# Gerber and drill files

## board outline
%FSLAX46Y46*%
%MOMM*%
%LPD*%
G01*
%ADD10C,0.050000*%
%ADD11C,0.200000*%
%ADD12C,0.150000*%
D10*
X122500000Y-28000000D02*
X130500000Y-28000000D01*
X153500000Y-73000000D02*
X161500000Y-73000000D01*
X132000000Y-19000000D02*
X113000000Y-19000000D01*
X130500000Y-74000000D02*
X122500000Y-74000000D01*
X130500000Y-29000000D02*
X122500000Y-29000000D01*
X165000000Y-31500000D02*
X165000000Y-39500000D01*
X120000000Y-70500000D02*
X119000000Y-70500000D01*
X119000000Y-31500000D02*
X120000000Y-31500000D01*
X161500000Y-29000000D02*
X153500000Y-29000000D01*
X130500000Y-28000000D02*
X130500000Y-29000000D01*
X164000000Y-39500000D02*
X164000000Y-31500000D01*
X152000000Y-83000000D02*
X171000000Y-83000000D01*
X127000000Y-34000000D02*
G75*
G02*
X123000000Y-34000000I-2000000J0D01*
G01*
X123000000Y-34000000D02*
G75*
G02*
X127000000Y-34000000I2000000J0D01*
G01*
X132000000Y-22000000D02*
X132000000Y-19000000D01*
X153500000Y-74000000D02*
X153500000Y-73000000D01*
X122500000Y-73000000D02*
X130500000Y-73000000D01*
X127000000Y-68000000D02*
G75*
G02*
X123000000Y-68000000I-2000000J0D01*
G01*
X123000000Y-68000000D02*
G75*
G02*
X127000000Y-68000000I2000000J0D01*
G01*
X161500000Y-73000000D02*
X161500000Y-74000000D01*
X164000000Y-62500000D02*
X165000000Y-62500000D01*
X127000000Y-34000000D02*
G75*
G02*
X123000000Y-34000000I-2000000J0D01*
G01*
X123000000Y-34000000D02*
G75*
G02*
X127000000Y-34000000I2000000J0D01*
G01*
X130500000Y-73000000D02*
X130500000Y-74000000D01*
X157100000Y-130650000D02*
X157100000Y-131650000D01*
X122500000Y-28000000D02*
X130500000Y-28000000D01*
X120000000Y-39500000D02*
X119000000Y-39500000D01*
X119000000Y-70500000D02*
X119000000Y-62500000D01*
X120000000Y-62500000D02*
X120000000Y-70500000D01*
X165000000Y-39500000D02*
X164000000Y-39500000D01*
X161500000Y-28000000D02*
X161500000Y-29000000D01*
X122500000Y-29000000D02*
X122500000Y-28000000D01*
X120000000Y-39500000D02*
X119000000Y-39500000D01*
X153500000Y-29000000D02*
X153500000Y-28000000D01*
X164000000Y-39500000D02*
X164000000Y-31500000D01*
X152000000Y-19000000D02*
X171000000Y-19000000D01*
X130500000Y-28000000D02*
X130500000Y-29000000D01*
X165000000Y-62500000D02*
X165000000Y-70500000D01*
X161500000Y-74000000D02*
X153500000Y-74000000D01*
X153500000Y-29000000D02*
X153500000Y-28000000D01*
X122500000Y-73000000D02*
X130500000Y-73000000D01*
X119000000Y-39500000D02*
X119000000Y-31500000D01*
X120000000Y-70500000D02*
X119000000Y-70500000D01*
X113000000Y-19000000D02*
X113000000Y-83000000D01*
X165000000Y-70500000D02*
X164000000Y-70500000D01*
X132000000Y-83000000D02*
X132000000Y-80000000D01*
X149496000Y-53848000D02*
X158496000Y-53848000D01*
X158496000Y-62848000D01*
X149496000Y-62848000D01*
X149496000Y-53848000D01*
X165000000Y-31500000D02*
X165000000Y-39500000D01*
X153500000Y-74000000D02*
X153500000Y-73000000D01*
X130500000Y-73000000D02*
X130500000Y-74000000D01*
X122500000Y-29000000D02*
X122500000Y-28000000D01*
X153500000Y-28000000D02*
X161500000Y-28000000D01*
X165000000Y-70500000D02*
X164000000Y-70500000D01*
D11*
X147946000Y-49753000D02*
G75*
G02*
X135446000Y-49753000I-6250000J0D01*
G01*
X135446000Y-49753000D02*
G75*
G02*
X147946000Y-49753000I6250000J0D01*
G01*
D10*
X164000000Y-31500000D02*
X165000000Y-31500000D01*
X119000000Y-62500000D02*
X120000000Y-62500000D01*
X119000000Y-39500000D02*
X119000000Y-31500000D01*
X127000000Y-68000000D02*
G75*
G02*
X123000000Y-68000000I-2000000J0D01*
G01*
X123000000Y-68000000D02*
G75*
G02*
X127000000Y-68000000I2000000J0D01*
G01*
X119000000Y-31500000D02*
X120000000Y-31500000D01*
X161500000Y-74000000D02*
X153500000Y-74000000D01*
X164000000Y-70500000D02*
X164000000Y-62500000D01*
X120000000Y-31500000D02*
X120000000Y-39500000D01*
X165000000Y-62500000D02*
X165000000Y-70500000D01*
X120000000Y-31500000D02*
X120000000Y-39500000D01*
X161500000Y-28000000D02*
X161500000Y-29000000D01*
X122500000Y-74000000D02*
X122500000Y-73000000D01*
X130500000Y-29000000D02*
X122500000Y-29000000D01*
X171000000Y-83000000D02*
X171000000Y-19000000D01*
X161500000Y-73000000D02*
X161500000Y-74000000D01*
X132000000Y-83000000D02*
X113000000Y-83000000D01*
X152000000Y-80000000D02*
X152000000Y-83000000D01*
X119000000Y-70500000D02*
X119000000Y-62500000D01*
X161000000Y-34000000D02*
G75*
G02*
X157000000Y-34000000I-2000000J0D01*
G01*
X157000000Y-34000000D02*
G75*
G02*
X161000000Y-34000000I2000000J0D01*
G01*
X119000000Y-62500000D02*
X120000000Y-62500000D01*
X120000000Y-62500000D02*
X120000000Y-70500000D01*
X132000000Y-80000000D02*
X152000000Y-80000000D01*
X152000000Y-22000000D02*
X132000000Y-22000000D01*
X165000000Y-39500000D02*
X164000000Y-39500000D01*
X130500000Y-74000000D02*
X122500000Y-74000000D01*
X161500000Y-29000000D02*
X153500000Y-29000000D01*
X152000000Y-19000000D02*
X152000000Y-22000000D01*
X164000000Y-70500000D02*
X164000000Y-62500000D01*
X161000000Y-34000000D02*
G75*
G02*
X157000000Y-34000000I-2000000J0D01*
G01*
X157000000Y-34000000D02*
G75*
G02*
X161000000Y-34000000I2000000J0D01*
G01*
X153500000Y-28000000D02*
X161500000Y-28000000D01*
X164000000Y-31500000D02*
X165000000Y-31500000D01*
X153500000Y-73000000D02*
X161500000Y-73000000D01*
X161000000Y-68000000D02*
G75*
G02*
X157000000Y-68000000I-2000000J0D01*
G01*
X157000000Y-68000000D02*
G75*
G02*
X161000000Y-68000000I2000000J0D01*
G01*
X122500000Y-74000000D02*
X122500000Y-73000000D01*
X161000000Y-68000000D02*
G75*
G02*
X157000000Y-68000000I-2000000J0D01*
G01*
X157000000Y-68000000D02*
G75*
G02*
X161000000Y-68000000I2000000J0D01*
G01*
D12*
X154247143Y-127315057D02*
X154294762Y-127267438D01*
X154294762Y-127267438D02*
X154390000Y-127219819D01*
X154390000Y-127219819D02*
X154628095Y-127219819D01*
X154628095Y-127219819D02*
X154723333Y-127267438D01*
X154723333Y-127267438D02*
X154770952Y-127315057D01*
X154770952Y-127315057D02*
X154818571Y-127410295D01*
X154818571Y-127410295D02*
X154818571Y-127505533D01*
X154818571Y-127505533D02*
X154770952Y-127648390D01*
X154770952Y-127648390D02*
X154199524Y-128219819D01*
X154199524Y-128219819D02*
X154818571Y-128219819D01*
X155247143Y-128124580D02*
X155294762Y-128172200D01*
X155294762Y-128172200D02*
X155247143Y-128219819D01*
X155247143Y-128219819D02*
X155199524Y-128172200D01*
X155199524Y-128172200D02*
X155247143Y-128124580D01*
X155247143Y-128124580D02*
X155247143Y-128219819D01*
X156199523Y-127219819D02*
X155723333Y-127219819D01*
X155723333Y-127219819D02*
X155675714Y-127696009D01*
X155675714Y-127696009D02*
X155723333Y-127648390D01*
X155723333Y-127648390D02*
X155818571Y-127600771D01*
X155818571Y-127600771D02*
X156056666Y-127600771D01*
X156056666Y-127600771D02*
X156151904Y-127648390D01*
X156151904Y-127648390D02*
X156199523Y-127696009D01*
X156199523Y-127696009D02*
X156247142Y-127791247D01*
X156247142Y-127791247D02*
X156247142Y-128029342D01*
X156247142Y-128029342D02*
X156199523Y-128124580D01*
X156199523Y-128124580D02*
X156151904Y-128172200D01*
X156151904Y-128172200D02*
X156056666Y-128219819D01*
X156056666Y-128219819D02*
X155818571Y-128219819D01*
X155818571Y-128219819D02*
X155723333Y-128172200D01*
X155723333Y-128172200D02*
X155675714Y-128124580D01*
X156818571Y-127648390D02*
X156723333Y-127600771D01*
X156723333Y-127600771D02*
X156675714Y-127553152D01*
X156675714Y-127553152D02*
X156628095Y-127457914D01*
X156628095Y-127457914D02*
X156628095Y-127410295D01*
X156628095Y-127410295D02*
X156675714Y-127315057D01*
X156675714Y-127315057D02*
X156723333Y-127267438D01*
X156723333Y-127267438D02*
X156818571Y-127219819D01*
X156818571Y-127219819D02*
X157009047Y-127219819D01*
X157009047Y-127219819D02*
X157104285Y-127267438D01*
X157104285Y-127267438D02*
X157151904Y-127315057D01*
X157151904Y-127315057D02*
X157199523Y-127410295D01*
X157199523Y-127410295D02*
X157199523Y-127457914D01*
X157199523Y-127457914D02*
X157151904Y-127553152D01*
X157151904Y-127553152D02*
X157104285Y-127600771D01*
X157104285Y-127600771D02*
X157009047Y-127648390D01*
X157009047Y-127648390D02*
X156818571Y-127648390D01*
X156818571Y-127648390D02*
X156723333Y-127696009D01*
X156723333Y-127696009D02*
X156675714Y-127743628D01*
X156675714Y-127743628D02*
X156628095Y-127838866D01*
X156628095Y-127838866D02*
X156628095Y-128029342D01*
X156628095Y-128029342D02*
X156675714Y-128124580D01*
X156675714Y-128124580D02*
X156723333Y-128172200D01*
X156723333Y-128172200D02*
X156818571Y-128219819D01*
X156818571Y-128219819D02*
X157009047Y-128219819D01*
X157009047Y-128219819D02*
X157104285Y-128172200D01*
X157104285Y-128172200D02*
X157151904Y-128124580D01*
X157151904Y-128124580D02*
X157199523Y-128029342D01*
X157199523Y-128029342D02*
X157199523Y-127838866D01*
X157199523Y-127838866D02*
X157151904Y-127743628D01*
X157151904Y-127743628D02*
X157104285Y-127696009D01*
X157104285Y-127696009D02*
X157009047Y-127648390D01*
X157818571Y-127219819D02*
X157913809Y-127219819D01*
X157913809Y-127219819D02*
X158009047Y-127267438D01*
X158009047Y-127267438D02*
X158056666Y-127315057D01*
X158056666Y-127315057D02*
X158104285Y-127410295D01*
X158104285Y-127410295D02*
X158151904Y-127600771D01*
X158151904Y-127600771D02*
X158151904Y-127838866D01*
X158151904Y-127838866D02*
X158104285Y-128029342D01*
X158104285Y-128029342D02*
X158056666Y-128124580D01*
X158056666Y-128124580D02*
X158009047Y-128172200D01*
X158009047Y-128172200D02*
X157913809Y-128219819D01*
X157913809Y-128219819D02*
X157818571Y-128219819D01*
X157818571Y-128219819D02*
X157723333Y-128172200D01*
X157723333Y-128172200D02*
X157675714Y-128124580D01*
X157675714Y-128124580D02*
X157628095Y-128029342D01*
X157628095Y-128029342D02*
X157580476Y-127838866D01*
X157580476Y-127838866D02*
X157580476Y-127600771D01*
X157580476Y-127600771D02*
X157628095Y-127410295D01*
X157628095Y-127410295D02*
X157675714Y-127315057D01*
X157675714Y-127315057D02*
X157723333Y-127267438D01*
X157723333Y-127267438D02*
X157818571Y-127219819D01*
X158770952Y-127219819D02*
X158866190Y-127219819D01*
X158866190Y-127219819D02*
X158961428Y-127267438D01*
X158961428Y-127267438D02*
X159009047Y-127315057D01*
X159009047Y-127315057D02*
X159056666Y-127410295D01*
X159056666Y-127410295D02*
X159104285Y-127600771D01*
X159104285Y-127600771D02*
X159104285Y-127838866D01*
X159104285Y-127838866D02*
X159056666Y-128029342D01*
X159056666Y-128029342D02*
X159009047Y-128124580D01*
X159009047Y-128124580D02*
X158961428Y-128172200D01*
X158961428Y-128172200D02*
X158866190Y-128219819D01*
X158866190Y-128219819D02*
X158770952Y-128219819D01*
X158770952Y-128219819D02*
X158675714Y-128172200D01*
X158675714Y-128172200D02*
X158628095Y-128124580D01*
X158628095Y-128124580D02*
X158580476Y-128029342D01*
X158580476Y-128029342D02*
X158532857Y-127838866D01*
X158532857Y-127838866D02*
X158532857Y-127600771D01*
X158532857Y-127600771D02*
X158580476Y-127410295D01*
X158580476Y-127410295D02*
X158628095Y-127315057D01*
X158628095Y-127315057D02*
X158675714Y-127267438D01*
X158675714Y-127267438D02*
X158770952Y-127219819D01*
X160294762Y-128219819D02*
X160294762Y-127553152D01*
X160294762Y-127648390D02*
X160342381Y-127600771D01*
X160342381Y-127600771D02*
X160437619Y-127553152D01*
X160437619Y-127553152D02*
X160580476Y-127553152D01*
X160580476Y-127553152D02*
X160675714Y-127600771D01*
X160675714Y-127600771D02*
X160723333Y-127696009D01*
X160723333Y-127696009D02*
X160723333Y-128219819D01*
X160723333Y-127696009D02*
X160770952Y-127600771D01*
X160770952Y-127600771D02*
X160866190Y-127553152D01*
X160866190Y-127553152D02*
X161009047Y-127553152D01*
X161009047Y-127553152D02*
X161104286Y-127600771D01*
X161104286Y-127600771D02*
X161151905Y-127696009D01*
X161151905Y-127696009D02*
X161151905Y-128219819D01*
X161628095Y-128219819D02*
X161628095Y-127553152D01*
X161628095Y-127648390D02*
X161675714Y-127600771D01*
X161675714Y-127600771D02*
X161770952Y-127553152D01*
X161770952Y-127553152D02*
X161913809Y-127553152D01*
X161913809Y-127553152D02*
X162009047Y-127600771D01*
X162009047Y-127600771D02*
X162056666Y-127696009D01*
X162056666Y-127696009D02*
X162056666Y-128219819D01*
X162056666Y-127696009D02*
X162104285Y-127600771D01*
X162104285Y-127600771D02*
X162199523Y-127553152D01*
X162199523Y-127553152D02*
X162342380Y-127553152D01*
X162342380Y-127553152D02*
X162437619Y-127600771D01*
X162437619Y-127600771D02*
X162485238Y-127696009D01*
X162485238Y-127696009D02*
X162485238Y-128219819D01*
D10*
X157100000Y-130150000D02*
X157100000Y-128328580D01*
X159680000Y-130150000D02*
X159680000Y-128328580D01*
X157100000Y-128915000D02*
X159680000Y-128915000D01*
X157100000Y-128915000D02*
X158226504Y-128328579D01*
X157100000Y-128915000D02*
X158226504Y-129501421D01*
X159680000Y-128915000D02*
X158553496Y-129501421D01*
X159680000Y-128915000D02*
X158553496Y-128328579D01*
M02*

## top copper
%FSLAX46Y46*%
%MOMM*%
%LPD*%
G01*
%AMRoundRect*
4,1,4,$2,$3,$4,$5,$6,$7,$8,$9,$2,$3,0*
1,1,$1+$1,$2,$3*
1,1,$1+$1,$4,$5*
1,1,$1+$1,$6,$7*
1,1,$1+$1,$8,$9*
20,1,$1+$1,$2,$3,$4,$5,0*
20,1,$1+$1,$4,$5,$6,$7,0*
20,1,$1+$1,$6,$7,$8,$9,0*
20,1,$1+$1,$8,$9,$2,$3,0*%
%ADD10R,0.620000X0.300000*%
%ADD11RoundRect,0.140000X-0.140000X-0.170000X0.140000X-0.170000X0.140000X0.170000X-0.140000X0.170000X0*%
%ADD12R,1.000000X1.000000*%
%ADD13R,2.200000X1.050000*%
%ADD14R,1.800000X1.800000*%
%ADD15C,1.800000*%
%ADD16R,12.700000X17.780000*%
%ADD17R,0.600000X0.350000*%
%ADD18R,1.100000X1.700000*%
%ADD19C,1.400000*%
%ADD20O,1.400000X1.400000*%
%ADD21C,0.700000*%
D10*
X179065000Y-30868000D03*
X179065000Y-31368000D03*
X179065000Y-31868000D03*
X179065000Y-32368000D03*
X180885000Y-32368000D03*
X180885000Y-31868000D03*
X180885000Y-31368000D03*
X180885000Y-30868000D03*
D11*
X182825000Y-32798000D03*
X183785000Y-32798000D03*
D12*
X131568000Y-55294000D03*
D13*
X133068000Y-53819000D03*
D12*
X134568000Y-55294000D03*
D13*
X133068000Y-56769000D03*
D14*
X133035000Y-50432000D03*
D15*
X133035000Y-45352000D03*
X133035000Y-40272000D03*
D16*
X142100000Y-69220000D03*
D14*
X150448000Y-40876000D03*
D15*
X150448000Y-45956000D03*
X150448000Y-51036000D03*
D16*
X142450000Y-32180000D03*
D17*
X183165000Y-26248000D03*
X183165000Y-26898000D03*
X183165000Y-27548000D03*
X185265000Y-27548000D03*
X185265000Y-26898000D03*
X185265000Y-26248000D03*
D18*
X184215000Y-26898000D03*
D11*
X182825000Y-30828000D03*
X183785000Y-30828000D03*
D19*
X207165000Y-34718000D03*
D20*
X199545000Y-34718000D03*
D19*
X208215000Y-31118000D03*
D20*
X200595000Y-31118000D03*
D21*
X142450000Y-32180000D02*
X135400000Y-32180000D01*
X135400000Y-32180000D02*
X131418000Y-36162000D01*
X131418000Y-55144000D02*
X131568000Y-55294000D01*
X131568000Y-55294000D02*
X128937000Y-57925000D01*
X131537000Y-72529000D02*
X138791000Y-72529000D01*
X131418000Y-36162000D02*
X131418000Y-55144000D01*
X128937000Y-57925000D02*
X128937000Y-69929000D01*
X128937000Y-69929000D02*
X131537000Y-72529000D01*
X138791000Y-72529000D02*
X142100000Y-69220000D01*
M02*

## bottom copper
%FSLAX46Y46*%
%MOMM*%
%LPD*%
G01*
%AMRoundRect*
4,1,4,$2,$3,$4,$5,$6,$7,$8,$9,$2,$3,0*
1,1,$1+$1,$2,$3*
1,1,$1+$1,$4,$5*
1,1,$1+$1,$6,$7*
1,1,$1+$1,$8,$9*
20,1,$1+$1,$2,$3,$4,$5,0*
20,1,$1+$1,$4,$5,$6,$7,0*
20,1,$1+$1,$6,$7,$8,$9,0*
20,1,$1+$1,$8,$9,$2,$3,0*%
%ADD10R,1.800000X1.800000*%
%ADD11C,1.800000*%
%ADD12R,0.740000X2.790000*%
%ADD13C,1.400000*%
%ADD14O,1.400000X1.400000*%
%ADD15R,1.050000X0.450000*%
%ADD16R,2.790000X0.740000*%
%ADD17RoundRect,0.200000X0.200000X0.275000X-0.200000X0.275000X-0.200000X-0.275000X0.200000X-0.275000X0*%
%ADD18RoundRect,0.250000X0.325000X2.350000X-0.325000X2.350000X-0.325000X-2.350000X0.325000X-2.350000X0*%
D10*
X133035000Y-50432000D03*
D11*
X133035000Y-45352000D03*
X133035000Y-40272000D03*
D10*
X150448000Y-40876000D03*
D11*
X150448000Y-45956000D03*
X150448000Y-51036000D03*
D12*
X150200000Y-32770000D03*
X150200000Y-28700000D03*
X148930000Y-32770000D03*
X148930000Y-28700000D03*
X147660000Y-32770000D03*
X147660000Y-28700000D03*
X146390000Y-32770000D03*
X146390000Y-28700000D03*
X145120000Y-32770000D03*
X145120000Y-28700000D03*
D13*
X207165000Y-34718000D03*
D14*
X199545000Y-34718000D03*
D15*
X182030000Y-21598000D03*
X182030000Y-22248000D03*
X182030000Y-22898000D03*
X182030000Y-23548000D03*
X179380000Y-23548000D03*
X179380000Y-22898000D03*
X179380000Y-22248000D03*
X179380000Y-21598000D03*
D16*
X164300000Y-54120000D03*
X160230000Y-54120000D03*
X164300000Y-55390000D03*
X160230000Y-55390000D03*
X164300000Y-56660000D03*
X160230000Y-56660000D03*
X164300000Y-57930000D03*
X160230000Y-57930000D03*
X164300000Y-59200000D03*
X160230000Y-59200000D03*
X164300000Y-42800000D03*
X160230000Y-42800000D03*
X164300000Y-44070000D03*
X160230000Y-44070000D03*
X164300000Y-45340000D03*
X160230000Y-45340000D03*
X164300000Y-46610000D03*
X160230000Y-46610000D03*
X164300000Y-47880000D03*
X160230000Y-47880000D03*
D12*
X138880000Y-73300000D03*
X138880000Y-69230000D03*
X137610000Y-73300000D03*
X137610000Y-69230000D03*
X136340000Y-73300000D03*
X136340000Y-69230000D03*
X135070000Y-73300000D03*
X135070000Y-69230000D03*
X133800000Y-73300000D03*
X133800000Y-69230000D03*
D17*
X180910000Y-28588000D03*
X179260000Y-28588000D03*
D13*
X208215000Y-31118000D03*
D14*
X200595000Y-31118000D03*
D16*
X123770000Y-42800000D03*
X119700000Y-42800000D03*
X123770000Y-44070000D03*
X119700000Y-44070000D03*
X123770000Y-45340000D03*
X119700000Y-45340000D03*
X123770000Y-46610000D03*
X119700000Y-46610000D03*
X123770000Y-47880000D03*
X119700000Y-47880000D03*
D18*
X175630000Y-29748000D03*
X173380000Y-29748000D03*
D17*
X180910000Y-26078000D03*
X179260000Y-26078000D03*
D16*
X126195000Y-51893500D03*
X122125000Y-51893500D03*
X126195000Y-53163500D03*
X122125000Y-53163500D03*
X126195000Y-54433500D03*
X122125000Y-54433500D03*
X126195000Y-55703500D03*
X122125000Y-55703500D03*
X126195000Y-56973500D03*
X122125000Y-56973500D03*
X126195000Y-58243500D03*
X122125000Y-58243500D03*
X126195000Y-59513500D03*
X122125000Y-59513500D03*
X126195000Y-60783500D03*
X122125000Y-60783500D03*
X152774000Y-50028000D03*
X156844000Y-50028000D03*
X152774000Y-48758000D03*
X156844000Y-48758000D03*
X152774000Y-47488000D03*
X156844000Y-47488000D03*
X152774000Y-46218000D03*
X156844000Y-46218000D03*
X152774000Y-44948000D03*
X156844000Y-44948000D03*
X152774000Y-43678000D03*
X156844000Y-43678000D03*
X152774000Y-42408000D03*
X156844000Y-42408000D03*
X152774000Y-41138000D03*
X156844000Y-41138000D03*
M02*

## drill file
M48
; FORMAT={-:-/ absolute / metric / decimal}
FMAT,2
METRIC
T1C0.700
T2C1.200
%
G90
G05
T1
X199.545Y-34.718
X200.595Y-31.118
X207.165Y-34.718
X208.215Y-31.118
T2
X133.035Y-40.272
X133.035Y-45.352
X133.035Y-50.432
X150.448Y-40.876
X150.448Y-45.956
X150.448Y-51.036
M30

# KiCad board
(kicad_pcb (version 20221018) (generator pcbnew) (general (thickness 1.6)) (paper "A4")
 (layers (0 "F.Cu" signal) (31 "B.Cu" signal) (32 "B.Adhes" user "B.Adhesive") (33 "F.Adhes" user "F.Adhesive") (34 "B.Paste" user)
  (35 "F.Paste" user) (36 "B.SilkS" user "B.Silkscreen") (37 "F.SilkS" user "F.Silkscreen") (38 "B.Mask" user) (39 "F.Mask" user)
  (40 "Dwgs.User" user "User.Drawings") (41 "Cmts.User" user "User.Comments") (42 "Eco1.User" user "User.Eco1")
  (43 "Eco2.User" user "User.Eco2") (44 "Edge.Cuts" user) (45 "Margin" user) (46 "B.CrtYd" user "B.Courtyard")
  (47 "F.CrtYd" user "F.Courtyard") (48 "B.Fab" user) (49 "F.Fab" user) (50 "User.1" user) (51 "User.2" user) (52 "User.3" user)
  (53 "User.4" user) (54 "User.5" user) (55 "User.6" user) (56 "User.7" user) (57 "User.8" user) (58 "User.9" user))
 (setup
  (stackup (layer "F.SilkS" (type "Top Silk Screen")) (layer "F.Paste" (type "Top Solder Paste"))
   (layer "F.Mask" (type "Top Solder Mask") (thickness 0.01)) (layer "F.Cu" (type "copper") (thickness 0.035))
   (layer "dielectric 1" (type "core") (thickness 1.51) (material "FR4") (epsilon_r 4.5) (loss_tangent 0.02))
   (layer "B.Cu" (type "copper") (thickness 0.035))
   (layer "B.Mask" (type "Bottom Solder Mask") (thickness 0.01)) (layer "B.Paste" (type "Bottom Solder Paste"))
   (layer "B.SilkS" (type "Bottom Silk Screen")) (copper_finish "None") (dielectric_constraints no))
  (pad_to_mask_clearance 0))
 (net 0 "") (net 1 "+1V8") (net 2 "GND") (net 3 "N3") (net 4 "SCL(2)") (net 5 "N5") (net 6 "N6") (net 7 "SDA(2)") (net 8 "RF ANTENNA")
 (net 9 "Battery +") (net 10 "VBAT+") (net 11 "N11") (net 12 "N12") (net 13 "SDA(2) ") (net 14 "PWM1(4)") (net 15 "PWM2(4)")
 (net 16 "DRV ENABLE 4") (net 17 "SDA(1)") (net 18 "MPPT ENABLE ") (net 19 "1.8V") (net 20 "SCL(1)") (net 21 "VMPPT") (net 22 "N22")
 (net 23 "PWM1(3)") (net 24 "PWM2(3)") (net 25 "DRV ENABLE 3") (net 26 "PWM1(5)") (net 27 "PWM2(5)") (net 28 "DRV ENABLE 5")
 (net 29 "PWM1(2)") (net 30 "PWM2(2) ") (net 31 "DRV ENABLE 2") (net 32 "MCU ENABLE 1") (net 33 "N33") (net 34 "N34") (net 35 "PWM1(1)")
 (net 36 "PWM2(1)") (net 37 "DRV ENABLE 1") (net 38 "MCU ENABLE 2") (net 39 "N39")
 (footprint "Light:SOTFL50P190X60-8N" (layer "F.Cu") (at 179.975 31.618)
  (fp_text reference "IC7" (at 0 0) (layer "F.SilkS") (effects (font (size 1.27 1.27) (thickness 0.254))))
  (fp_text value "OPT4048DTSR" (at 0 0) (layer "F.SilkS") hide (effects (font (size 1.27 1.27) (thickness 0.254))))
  (pad "1" smd rect (at -0.91 -0.75 90) (size 0.3 0.62) (layers "F.Cu" "F.Paste" "F.Mask") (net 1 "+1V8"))
  (pad "2" smd rect (at -0.91 -0.25 90) (size 0.3 0.62) (layers "F.Cu" "F.Paste" "F.Mask") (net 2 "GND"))
  (pad "3" smd rect (at -0.91 0.25 90) (size 0.3 0.62) (layers "F.Cu" "F.Paste" "F.Mask") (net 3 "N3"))
  (pad "4" smd rect (at -0.91 0.75 90) (size 0.3 0.62) (layers "F.Cu" "F.Paste" "F.Mask") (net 2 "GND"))
  (pad "5" smd rect (at 0.91 0.75 90) (size 0.3 0.62) (layers "F.Cu" "F.Paste" "F.Mask") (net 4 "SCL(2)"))
  (pad "6" smd rect (at 0.91 0.25 90) (size 0.3 0.62) (layers "F.Cu" "F.Paste" "F.Mask") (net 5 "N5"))
  (pad "7" smd rect (at 0.91 -0.25 90) (size 0.3 0.62) (layers "F.Cu" "F.Paste" "F.Mask") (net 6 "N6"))
  (pad "8" smd rect (at 0.91 -0.75 90) (size 0.3 0.62) (layers "F.Cu" "F.Paste" "F.Mask") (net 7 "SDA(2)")))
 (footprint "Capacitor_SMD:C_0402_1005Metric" (layer "F.Cu") (at 183.305 32.798)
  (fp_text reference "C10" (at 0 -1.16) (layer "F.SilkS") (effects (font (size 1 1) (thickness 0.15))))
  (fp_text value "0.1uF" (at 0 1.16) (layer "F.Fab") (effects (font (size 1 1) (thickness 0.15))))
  (pad "1" smd roundrect (at -0.48 0) (size 0.56 0.62) (layers "F.Cu" "F.Paste" "F.Mask") (roundrect_rratio 0.25) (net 2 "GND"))
  (pad "2" smd roundrect (at 0.48 0) (size 0.56 0.62) (layers "F.Cu" "F.Paste" "F.Mask") (roundrect_rratio 0.25) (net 1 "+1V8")))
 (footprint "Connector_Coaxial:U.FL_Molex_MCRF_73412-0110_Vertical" (layer "F.Cu") (at 133.068 55.294 -90)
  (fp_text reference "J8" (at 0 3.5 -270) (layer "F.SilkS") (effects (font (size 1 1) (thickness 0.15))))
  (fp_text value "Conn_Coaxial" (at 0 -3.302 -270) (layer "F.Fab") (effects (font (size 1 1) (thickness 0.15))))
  (pad "1" smd rect (at 0 1.5 270) (size 1 1) (layers "F.Cu" "F.Paste" "F.Mask") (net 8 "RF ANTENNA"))
  (pad "2" smd rect (at -1.475 0 270) (size 1.05 2.2) (layers "F.Cu" "F.Paste" "F.Mask") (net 2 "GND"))
  (pad "2" smd rect (at 0 -1.5 270) (size 1 1) (layers "F.Cu" "F.Paste" "F.Mask") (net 2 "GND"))
  (pad "2" smd rect (at 1.475 0 270) (size 1.05 2.2) (layers "F.Cu" "F.Paste" "F.Mask") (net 2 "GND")))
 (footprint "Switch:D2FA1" (layer "F.Cu") (at 133.035 50.432 90)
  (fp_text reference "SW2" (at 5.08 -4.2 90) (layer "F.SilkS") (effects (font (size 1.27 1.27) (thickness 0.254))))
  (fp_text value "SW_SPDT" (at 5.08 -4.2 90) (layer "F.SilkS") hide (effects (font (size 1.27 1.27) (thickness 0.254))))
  (pad "1" thru_hole rect (at 0 0 90) (size 1.8 1.8) (drill 1.2) (layers "*.Cu" "*.Mask") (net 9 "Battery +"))
  (pad "2" thru_hole circle (at 5.08 0 90) (size 1.8 1.8) (drill 1.2) (layers "*.Cu" "*.Mask") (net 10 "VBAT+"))
  (pad "3" thru_hole circle (at 10.16 0 90) (size 1.8 1.8) (drill 1.2) (layers "*.Cu" "*.Mask") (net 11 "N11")))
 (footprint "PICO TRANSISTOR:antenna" (layer "F.Cu") (at 142.1 67.95 -90)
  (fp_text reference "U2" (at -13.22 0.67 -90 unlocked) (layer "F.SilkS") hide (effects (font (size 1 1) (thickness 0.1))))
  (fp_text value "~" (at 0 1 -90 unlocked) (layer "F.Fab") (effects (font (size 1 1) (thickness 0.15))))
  (pad "1" smd rect (at 1.27 0 270) (size 17.78 12.7) (layers "F.Cu" "F.Paste" "F.Mask") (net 8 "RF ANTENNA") (thermal_bridge_angle 45)))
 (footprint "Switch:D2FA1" (layer "F.Cu") (at 150.448 40.876 -90)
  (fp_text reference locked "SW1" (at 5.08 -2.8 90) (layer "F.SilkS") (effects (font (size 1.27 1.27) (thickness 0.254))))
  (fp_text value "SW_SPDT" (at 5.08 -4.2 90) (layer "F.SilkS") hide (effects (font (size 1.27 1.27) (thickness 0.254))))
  (pad "1" thru_hole rect (at 0 0 270) (size 1.8 1.8) (drill 1.2) (layers "*.Cu" "*.Mask") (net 9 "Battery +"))
  (pad "2" thru_hole circle (at 5.08 0 270) (size 1.8 1.8) (drill 1.2) (layers "*.Cu" "*.Mask") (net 10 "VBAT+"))
  (pad "3" thru_hole circle (at 10.16 0 270) (size 1.8 1.8) (drill 1.2) (layers "*.Cu" "*.Mask") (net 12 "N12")))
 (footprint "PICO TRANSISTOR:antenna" (layer "F.Cu") (at 142.45 33.45 90)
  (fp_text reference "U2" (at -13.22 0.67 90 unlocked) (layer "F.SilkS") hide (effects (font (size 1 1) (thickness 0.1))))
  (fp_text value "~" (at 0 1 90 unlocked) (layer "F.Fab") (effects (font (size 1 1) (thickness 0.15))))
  (pad "1" smd rect (at 1.27 0 90) (size 17.78 12.7) (layers "F.Cu" "F.Paste" "F.Mask") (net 8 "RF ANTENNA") (thermal_bridge_angle 45)))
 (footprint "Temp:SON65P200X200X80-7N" (layer "F.Cu") (at 184.215 26.898)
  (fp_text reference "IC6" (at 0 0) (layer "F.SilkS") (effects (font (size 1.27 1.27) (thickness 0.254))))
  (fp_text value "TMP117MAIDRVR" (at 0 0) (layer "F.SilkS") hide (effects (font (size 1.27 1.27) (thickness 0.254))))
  (pad "1" smd rect (at -1.05 -0.65 90) (size 0.35 0.6) (layers "F.Cu" "F.Paste" "F.Mask") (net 4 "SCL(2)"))
  (pad "2" smd rect (at -1.05 0 90) (size 0.35 0.6) (layers "F.Cu" "F.Paste" "F.Mask") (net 2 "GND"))
  (pad "3" smd rect (at -1.05 0.65 90) (size 0.35 0.6) (layers "F.Cu" "F.Paste" "F.Mask") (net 2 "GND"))
  (pad "4" smd rect (at 1.05 0.65 90) (size 0.35 0.6) (layers "F.Cu" "F.Paste" "F.Mask") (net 2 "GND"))
  (pad "5" smd rect (at 1.05 0 90) (size 0.35 0.6) (layers "F.Cu" "F.Paste" "F.Mask") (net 1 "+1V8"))
  (pad "6" smd rect (at 1.05 -0.65 90) (size 0.35 0.6) (layers "F.Cu" "F.Paste" "F.Mask") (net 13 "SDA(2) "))
  (pad "7" smd rect (at 0 0) (size 1.1 1.7) (layers "F.Cu" "F.Paste" "F.Mask") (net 2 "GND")))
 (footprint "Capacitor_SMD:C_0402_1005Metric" (layer "F.Cu") (at 183.305 30.828)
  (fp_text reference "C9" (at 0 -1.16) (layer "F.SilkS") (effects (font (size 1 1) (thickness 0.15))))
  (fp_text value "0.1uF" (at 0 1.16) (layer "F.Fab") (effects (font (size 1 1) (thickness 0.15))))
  (pad "1" smd roundrect (at -0.48 0) (size 0.56 0.62) (layers "F.Cu" "F.Paste" "F.Mask") (roundrect_rratio 0.25) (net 2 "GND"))
  (pad "2" smd roundrect (at 0.48 0) (size 0.56 0.62) (layers "F.Cu" "F.Paste" "F.Mask") (roundrect_rratio 0.25) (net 1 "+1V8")))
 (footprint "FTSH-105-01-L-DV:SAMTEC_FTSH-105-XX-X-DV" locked (layer "B.Cu") (at 147.66 30.735 180)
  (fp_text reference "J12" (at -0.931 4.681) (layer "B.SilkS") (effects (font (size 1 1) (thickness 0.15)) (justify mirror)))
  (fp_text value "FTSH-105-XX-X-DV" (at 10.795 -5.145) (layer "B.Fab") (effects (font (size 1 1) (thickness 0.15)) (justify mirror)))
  (pad "01" smd rect locked (at -2.54 -2.035 180) (size 0.74 2.79) (layers "B.Cu" "B.Paste" "B.Mask") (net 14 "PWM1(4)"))
  (pad "02" smd rect locked (at -2.54 2.035 180) (size 0.74 2.79) (layers "B.Cu" "B.Paste" "B.Mask") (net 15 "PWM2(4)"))
  (pad "03" smd rect locked (at -1.27 -2.035 180) (size 0.74 2.79) (layers "B.Cu" "B.Paste" "B.Mask") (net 9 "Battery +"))
  (pad "04" smd rect locked (at -1.27 2.035 180) (size 0.74 2.79) (layers "B.Cu" "B.Paste" "B.Mask") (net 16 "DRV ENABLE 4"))
  (pad "05" smd rect locked (at 0 -2.035 180) (size 0.74 2.79) (layers "B.Cu" "B.Paste" "B.Mask") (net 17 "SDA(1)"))
  (pad "06" smd rect locked (at 0 2.035 180) (size 0.74 2.79) (layers "B.Cu" "B.Paste" "B.Mask") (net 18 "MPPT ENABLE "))
  (pad "07" smd rect locked (at 1.27 -2.035 180) (size 0.74 2.79) (layers "B.Cu" "B.Paste" "B.Mask") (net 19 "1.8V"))
  (pad "08" smd rect locked (at 1.27 2.035 180) (size 0.74 2.79) (layers "B.Cu" "B.Paste" "B.Mask") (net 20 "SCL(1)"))
  (pad "09" smd rect locked (at 2.54 -2.035 180) (size 0.74 2.79) (layers "B.Cu" "B.Paste" "B.Mask") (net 2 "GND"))
  (pad "10" smd rect locked (at 2.54 2.035 180) (size 0.74 2.79) (layers "B.Cu" "B.Paste" "B.Mask") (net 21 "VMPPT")))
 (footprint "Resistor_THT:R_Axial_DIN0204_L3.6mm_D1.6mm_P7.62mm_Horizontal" (layer "B.Cu") (at 207.165 34.718 180)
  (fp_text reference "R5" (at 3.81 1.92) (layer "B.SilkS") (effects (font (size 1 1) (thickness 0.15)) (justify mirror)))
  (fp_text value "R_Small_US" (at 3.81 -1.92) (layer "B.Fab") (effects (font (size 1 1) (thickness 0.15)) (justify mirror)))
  (pad "1" thru_hole circle (at 0 0 180) (size 1.4 1.4) (drill 0.7) (layers "*.Cu" "*.Mask") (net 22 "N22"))
  (pad "2" thru_hole oval (at 7.62 0 180) (size 1.4 1.4) (drill 0.7) (layers "*.Cu" "*.Mask") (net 2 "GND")))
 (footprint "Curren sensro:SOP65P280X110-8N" (layer "B.Cu") (at 180.705 22.573 180)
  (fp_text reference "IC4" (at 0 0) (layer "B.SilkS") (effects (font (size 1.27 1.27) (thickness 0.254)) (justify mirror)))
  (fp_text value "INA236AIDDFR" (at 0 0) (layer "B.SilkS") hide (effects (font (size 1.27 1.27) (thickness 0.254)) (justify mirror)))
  (pad "1" smd rect (at -1.325 0.975 90) (size 0.45 1.05) (layers "B.Cu" "B.Paste" "B.Mask") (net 21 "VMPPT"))
  (pad "2" smd rect (at -1.325 0.325 90) (size 0.45 1.05) (layers "B.Cu" "B.Paste" "B.Mask") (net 9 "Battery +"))
  (pad "3" smd rect (at -1.325 -0.325 90) (size 0.45 1.05) (layers "B.Cu" "B.Paste" "B.Mask") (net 2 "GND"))
  (pad "4" smd rect (at -1.325 -0.975 90) (size 0.45 1.05) (layers "B.Cu" "B.Paste" "B.Mask") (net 1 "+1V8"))
  (pad "5" smd rect (at 1.325 -0.975 90) (size 0.45 1.05) (layers "B.Cu" "B.Paste" "B.Mask") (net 20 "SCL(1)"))
  (pad "6" smd rect (at 1.325 -0.325 90) (size 0.45 1.05) (layers "B.Cu" "B.Paste" "B.Mask") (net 17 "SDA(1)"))
  (pad "7" smd rect (at 1.325 0.325 90) (size 0.45 1.05) (layers "B.Cu" "B.Paste" "B.Mask") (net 2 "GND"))
  (pad "8" smd rect (at 1.325 0.975 90) (size 0.45 1.05) (layers "B.Cu" "B.Paste" "B.Mask") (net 2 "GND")))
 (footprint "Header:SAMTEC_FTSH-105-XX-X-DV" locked (layer "B.Cu") (at 162.265 56.66 -90)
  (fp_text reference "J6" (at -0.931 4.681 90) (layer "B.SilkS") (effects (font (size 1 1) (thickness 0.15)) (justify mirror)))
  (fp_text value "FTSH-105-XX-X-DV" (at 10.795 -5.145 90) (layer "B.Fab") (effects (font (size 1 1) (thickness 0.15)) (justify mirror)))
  (pad "01" smd rect locked (at -2.54 -2.035 270) (size 0.74 2.79) (layers "B.Cu" "B.Paste" "B.Mask") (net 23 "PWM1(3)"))
  (pad "02" smd rect locked (at -2.54 2.035 270) (size 0.74 2.79) (layers "B.Cu" "B.Paste" "B.Mask") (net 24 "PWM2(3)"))
  (pad "03" smd rect locked (at -1.27 -2.035 270) (size 0.74 2.79) (layers "B.Cu" "B.Paste" "B.Mask") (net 9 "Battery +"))
  (pad "04" smd rect locked (at -1.27 2.035 270) (size 0.74 2.79) (layers "B.Cu" "B.Paste" "B.Mask") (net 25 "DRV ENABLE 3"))
  (pad "05" smd rect locked (at 0 -2.035 270) (size 0.74 2.79) (layers "B.Cu" "B.Paste" "B.Mask") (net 17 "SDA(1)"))
  (pad "06" smd rect locked (at 0 2.035 270) (size 0.74 2.79) (layers "B.Cu" "B.Paste" "B.Mask") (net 18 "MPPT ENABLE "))
  (pad "07" smd rect locked (at 1.27 -2.035 270) (size 0.74 2.79) (layers "B.Cu" "B.Paste" "B.Mask") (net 19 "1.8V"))
  (pad "08" smd rect locked (at 1.27 2.035 270) (size 0.74 2.79) (layers "B.Cu" "B.Paste" "B.Mask") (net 20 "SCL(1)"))
  (pad "09" smd rect locked (at 2.54 -2.035 270) (size 0.74 2.79) (layers "B.Cu" "B.Paste" "B.Mask") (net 2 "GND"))
  (pad "10" smd rect locked (at 2.54 2.035 270) (size 0.74 2.79) (layers "B.Cu" "B.Paste" "B.Mask") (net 21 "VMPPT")))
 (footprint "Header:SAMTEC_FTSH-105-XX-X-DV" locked (layer "B.Cu") (at 162.265 45.34 -90)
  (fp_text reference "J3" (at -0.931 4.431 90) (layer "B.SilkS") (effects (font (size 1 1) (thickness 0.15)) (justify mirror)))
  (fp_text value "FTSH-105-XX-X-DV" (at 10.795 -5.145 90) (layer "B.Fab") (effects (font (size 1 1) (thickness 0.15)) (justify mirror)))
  (pad "01" smd rect locked (at -2.54 -2.035 270) (size 0.74 2.79) (layers "B.Cu" "B.Paste" "B.Mask") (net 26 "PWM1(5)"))
  (pad "02" smd rect locked (at -2.54 2.035 270) (size 0.74 2.79) (layers "B.Cu" "B.Paste" "B.Mask") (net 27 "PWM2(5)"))
  (pad "03" smd rect locked (at -1.27 -2.035 270) (size 0.74 2.79) (layers "B.Cu" "B.Paste" "B.Mask") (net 9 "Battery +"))
  (pad "04" smd rect locked (at -1.27 2.035 270) (size 0.74 2.79) (layers "B.Cu" "B.Paste" "B.Mask") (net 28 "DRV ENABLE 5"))
  (pad "05" smd rect locked (at 0 -2.035 270) (size 0.74 2.79) (layers "B.Cu" "B.Paste" "B.Mask") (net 7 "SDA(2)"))
  (pad "06" smd rect locked (at 0 2.035 270) (size 0.74 2.79) (layers "B.Cu" "B.Paste" "B.Mask") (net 18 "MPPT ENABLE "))
  (pad "07" smd rect locked (at 1.27 -2.035 270) (size 0.74 2.79) (layers "B.Cu" "B.Paste" "B.Mask") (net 19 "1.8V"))
  (pad "08" smd rect locked (at 1.27 2.035 270) (size 0.74 2.79) (layers "B.Cu" "B.Paste" "B.Mask") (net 4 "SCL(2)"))
  (pad "09" smd rect locked (at 2.54 -2.035 270) (size 0.74 2.79) (layers "B.Cu" "B.Paste" "B.Mask") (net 2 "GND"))
  (pad "10" smd rect locked (at 2.54 2.035 270) (size 0.74 2.79) (layers "B.Cu" "B.Paste" "B.Mask") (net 21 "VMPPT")))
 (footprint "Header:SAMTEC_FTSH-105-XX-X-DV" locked (layer "B.Cu") (at 136.34 71.265 180)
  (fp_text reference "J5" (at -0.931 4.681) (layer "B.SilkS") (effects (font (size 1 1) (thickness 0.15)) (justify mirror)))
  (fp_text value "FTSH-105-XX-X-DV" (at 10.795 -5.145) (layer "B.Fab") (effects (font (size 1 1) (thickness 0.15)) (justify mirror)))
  (pad "01" smd rect locked (at -2.54 -2.035 180) (size 0.74 2.79) (layers "B.Cu" "B.Paste" "B.Mask") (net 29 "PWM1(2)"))
  (pad "02" smd rect locked (at -2.54 2.035 180) (size 0.74 2.79) (layers "B.Cu" "B.Paste" "B.Mask") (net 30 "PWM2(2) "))
  (pad "03" smd rect locked (at -1.27 -2.035 180) (size 0.74 2.79) (layers "B.Cu" "B.Paste" "B.Mask") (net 9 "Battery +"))
  (pad "04" smd rect locked (at -1.27 2.035 180) (size 0.74 2.79) (layers "B.Cu" "B.Paste" "B.Mask") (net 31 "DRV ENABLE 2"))
  (pad "05" smd rect locked (at 0 -2.035 180) (size 0.74 2.79) (layers "B.Cu" "B.Paste" "B.Mask") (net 17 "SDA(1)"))
  (pad "06" smd rect locked (at 0 2.035 180) (size 0.74 2.79) (layers "B.Cu" "B.Paste" "B.Mask") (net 18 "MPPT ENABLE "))
  (pad "07" smd rect locked (at 1.27 -2.035 180) (size 0.74 2.79) (layers "B.Cu" "B.Paste" "B.Mask") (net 19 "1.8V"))
  (pad "08" smd rect locked (at 1.27 2.035 180) (size 0.74 2.79) (layers "B.Cu" "B.Paste" "B.Mask") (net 20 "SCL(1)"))
  (pad "09" smd rect locked (at 2.54 -2.035 180) (size 0.74 2.79) (layers "B.Cu" "B.Paste" "B.Mask") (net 2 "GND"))
  (pad "10" smd rect locked (at 2.54 2.035 180) (size 0.74 2.79) (layers "B.Cu" "B.Paste" "B.Mask") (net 21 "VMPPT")))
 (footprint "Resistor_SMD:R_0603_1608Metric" (layer "B.Cu") (at 180.085 28.588 180)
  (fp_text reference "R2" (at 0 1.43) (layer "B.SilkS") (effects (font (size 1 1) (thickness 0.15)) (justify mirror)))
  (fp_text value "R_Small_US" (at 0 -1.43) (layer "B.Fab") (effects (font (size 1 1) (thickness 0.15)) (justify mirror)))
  (pad "1" smd roundrect (at -0.825 0 180) (size 0.8 0.95) (layers "B.Cu" "B.Paste" "B.Mask") (roundrect_rratio 0.25)
   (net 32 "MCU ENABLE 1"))
  (pad "2" smd roundrect (at 0.825 0 180) (size 0.8 0.95) (layers "B.Cu" "B.Paste" "B.Mask") (roundrect_rratio 0.25) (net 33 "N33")))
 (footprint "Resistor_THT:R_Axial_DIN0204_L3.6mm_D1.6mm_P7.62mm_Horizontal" (layer "B.Cu") (at 208.215 31.118 180)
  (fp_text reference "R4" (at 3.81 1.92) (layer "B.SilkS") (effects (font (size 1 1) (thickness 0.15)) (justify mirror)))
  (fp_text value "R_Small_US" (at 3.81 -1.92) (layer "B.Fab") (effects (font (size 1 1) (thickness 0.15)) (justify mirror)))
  (pad "1" thru_hole circle (at 0 0 180) (size 1.4 1.4) (drill 0.7) (layers "*.Cu" "*.Mask") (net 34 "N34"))
  (pad "2" thru_hole oval (at 7.62 0 180) (size 1.4 1.4) (drill 0.7) (layers "*.Cu" "*.Mask") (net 2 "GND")))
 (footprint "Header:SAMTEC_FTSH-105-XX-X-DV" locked (layer "B.Cu") (at 121.735 45.34 -90)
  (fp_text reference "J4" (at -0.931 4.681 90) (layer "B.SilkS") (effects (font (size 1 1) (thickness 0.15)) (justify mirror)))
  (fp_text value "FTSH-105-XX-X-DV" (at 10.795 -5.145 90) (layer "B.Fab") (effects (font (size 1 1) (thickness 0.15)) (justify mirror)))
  (pad "01" smd rect locked (at -2.54 -2.035 270) (size 0.74 2.79) (layers "B.Cu" "B.Paste" "B.Mask") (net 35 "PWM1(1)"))
  (pad "02" smd rect locked (at -2.54 2.035 270) (size 0.74 2.79) (layers "B.Cu" "B.Paste" "B.Mask") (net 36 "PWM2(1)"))
  (pad "03" smd rect locked (at -1.27 -2.035 270) (size 0.74 2.79) (layers "B.Cu" "B.Paste" "B.Mask") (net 9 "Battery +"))
  (pad "04" smd rect locked (at -1.27 2.035 270) (size 0.74 2.79) (layers "B.Cu" "B.Paste" "B.Mask") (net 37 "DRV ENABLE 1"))
  (pad "05" smd rect locked (at 0 -2.035 270) (size 0.74 2.79) (layers "B.Cu" "B.Paste" "B.Mask") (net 17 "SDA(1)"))
  (pad "06" smd rect locked (at 0 2.035 270) (size 0.74 2.79) (layers "B.Cu" "B.Paste" "B.Mask") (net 18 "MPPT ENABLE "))
  (pad "07" smd rect locked (at 1.27 -2.035 270) (size 0.74 2.79) (layers "B.Cu" "B.Paste" "B.Mask") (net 19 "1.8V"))
  (pad "08" smd rect locked (at 1.27 2.035 270) (size 0.74 2.79) (layers "B.Cu" "B.Paste" "B.Mask") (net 20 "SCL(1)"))
  (pad "09" smd rect locked (at 2.54 -2.035 270) (size 0.74 2.79) (layers "B.Cu" "B.Paste" "B.Mask") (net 2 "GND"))
  (pad "10" smd rect locked (at 2.54 2.035 270) (size 0.74 2.79) (layers "B.Cu" "B.Paste" "B.Mask") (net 21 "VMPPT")))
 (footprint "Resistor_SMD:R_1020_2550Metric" (layer "B.Cu") (at 174.505 29.748 180)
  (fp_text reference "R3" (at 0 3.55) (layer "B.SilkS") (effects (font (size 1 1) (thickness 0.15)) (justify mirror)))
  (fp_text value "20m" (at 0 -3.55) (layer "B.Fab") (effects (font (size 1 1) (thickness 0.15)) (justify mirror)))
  (pad "1" smd roundrect (at -1.125 0 180) (size 1.15 5.2) (layers "B.Cu" "B.Paste" "B.Mask") (roundrect_rratio 0.217391) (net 21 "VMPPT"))
  (pad "2" smd roundrect (at 1.125 0 180) (size 1.15 5.2) (layers "B.Cu" "B.Paste" "B.Mask") (roundrect_rratio 0.217391) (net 9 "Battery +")))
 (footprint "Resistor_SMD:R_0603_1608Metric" (layer "B.Cu") (at 180.085 26.078 180)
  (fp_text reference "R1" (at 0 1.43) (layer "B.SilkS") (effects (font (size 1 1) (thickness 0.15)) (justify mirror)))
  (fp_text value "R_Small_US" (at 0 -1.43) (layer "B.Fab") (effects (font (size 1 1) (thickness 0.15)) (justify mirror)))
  (pad "1" smd roundrect (at -0.825 0 180) (size 0.8 0.95) (layers "B.Cu" "B.Paste" "B.Mask") (roundrect_rratio 0.25)
   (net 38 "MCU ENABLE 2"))
  (pad "2" smd roundrect (at 0.825 0 180) (size 0.8 0.95) (layers "B.Cu" "B.Paste" "B.Mask") (roundrect_rratio 0.25) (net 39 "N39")))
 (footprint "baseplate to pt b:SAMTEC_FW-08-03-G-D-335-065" (layer "B.Cu") (at 124.16 56.3385 -90)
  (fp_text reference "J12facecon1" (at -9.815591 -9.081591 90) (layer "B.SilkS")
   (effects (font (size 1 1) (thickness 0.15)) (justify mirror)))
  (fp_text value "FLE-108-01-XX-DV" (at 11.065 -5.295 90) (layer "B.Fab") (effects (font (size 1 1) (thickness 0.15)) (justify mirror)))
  (pad "01" smd rect (at -4.445 -2.035 270) (size 0.74 2.79) (layers "B.Cu" "B.Paste" "B.Mask") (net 37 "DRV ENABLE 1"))
  (pad "02" smd rect (at -4.445 2.035 270) (size 0.74 2.79) (layers "B.Cu" "B.Paste" "B.Mask") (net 20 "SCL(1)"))
  (pad "03" smd rect (at -3.175 -2.035 270) (size 0.74 2.79) (layers "B.Cu" "B.Paste" "B.Mask") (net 31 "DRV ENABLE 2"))
  (pad "04" smd rect (at -3.175 2.035 270) (size 0.74 2.79) (layers "B.Cu" "B.Paste" "B.Mask") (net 17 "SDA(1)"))
  (pad "05" smd rect (at -1.905 -2.035 270) (size 0.74 2.79) (layers "B.Cu" "B.Paste" "B.Mask") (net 38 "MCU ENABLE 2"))
  (pad "06" smd rect (at -1.905 2.035 270) (size 0.74 2.79) (layers "B.Cu" "B.Paste" "B.Mask") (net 18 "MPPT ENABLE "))
  (pad "07" smd rect (at -0.635 -2.035 270) (size 0.74 2.79) (layers "B.Cu" "B.Paste" "B.Mask") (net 32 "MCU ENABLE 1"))
  (pad "08" smd rect (at -0.635 2.035 270) (size 0.74 2.79) (layers "B.Cu" "B.Paste" "B.Mask") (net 9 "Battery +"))
  (pad "09" smd rect (at 0.635 -2.035 270) (size 0.74 2.79) (layers "B.Cu" "B.Paste" "B.Mask") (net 30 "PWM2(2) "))
  (pad "10" smd rect (at 0.635 2.035 270) (size 0.74 2.79) (layers "B.Cu" "B.Paste" "B.Mask") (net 35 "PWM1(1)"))
  (pad "11" smd rect (at 1.905 -2.035 270) (size 0.74 2.79) (layers "B.Cu" "B.Paste" "B.Mask") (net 29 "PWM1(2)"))
  (pad "12" smd rect (at 1.905 2.035 270) (size 0.74 2.79) (layers "B.Cu" "B.Paste" "B.Mask") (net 36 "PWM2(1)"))
  (pad "13" smd rect (at 3.175 -2.035 270) (size 0.74 2.79) (layers "B.Cu" "B.Paste" "B.Mask") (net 9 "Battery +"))
  (pad "14" smd rect (at 3.175 2.035 270) (size 0.74 2.79) (layers "B.Cu" "B.Paste" "B.Mask") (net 19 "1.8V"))
  (pad "15" smd rect (at 4.445 -2.035 270) (size 0.74 2.79) (layers "B.Cu" "B.Paste" "B.Mask") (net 2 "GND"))
  (pad "16" smd rect (at 4.445 2.035 270) (size 0.74 2.79) (layers "B.Cu" "B.Paste" "B.Mask") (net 2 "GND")))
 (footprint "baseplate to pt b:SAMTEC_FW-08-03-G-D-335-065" (layer "B.Cu") (at 154.809 45.583 90)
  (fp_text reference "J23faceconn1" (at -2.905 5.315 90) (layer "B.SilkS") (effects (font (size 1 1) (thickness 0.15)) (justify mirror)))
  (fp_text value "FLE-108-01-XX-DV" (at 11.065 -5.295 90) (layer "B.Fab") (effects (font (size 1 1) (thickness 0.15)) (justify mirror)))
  (pad "01" smd rect (at -4.445 -2.035 90) (size 0.74 2.79) (layers "B.Cu" "B.Paste" "B.Mask") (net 15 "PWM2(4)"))
  (pad "02" smd rect (at -4.445 2.035 90) (size 0.74 2.79) (layers "B.Cu" "B.Paste" "B.Mask") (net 23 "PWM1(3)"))
  (pad "03" smd rect (at -3.175 -2.035 90) (size 0.74 2.79) (layers "B.Cu" "B.Paste" "B.Mask") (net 14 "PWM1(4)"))
  (pad "04" smd rect (at -3.175 2.035 90) (size 0.74 2.79) (layers "B.Cu" "B.Paste" "B.Mask") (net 24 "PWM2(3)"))
  (pad "05" smd rect (at -1.905 -2.035 90) (size 0.74 2.79) (layers "B.Cu" "B.Paste" "B.Mask") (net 10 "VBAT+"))
  (pad "06" smd rect (at -1.905 2.035 90) (size 0.74 2.79) (layers "B.Cu" "B.Paste" "B.Mask") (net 28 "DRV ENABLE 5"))
  (pad "07" smd rect (at -0.635 -2.035 90) (size 0.74 2.79) (layers "B.Cu" "B.Paste" "B.Mask") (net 21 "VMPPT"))
  (pad "08" smd rect (at -0.635 2.035 90) (size 0.74 2.79) (layers "B.Cu" "B.Paste" "B.Mask") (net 16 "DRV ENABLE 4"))
  (pad "09" smd rect (at 0.635 -2.035 90) (size 0.74 2.79) (layers "B.Cu" "B.Paste" "B.Mask") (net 26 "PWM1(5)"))
  (pad "10" smd rect (at 0.635 2.035 90) (size 0.74 2.79) (layers "B.Cu" "B.Paste" "B.Mask") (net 25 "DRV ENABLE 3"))
  (pad "11" smd rect (at 1.905 -2.035 90) (size 0.74 2.79) (layers "B.Cu" "B.Paste" "B.Mask") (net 19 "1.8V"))
  (pad "12" smd rect (at 1.905 2.035 90) (size 0.74 2.79) (layers "B.Cu" "B.Paste" "B.Mask") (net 4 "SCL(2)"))
  (pad "13" smd rect (at 3.175 -2.035 90) (size 0.74 2.79) (layers "B.Cu" "B.Paste" "B.Mask") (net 2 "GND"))
  (pad "14" smd rect (at 3.175 2.035 90) (size 0.74 2.79) (layers "B.Cu" "B.Paste" "B.Mask") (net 7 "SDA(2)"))
  (pad "15" smd rect (at 4.445 -2.035 90) (size 0.74 2.79) (layers "B.Cu" "B.Paste" "B.Mask") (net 2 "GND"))
  (pad "16" smd rect (at 4.445 2.035 90) (size 0.74 2.79) (layers "B.Cu" "B.Paste" "B.Mask") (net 27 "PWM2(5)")))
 (gr_line (start 122.5 28) (end 130.5 28) (stroke (width 0.05) (type default)) (layer "Edge.Cuts"))
 (gr_line (start 153.5 73) (end 161.5 73) (stroke (width 0.05) (type default)) (layer "Edge.Cuts"))
 (gr_line (start 132 19) (end 113 19) (stroke (width 0.05) (type default)) (layer "Edge.Cuts"))
 (gr_line (start 130.5 74) (end 122.5 74) (stroke (width 0.05) (type default)) (layer "Edge.Cuts"))
 (gr_line (start 130.5 29) (end 122.5 29) (stroke (width 0.05) (type default)) (layer "Edge.Cuts"))
 (gr_line (start 165 31.5) (end 165 39.5) (stroke (width 0.05) (type default)) (layer "Edge.Cuts"))
 (gr_line (start 120 70.5) (end 119 70.5) (stroke (width 0.05) (type default)) (layer "Edge.Cuts"))
 (gr_line (start 119 31.5) (end 120 31.5) (stroke (width 0.05) (type default)) (layer "Edge.Cuts"))
 (gr_line (start 161.5 29) (end 153.5 29) (stroke (width 0.05) (type default)) (layer "Edge.Cuts"))
 (gr_line (start 130.5 28) (end 130.5 29) (stroke (width 0.05) (type default)) (layer "Edge.Cuts"))
 (gr_line (start 164 39.5) (end 164 31.5) (stroke (width 0.05) (type default)) (layer "Edge.Cuts"))
 (gr_line (start 152 83) (end 171 83) (stroke (width 0.05) (type default)) (layer "Edge.Cuts"))
 (gr_circle (center 125 34) (end 127 34) (stroke (width 0.05) (type default)) (fill none) (layer "Edge.Cuts"))
 (gr_line (start 132 22) (end 132 19) (stroke (width 0.05) (type default)) (layer "Edge.Cuts"))
 (gr_line (start 153.5 74) (end 153.5 73) (stroke (width 0.05) (type default)) (layer "Edge.Cuts"))
 (gr_line (start 122.5 73) (end 130.5 73) (stroke (width 0.05) (type default)) (layer "Edge.Cuts"))
 (gr_circle (center 125 68) (end 125 66) (stroke (width 0.05) (type default)) (fill none) (layer "Edge.Cuts"))
 (gr_line (start 161.5 73) (end 161.5 74) (stroke (width 0.05) (type default)) (layer "Edge.Cuts"))
 (gr_line (start 164 62.5) (end 165 62.5) (stroke (width 0.05) (type default)) (layer "Edge.Cuts"))
 (gr_circle (center 125 34) (end 127 34) (stroke (width 0.05) (type default)) (fill none) (layer "Edge.Cuts"))
 (gr_line (start 130.5 73) (end 130.5 74) (stroke (width 0.05) (type default)) (layer "Edge.Cuts"))
 (gr_line (start 157.1 130.65) (end 157.1 131.65) (stroke (width 0.05) (type default)) (layer "Edge.Cuts"))
 (gr_line (start 122.5 28) (end 130.5 28) (stroke (width 0.05) (type default)) (layer "Edge.Cuts"))
 (gr_line (start 120 39.5) (end 119 39.5) (stroke (width 0.05) (type default)) (layer "Edge.Cuts"))
 (gr_line (start 119 70.5) (end 119 62.5) (stroke (width 0.05) (type default)) (layer "Edge.Cuts"))
 (gr_line (start 120 62.5) (end 120 70.5) (stroke (width 0.05) (type default)) (layer "Edge.Cuts"))
 (gr_line (start 165 39.5) (end 164 39.5) (stroke (width 0.05) (type default)) (layer "Edge.Cuts"))
 (gr_line (start 161.5 28) (end 161.5 29) (stroke (width 0.05) (type default)) (layer "Edge.Cuts"))
 (gr_line (start 122.5 29) (end 122.5 28) (stroke (width 0.05) (type default)) (layer "Edge.Cuts"))
 (gr_line (start 120 39.5) (end 119 39.5) (stroke (width 0.05) (type default)) (layer "Edge.Cuts"))
 (gr_line (start 153.5 29) (end 153.5 28) (stroke (width 0.05) (type default)) (layer "Edge.Cuts"))
 (gr_line (start 164 39.5) (end 164 31.5) (stroke (width 0.05) (type default)) (layer "Edge.Cuts"))
 (gr_line (start 152 19) (end 171 19) (stroke (width 0.05) (type default)) (layer "Edge.Cuts"))
 (gr_line (start 130.5 28) (end 130.5 29) (stroke (width 0.05) (type default)) (layer "Edge.Cuts"))
 (gr_line (start 165 62.5) (end 165 70.5) (stroke (width 0.05) (type default)) (layer "Edge.Cuts"))
 (gr_line (start 161.5 74) (end 153.5 74) (stroke (width 0.05) (type default)) (layer "Edge.Cuts"))
 (gr_line (start 153.5 29) (end 153.5 28) (stroke (width 0.05) (type default)) (layer "Edge.Cuts"))
 (gr_line (start 122.5 73) (end 130.5 73) (stroke (width 0.05) (type default)) (layer "Edge.Cuts"))
 (gr_line (start 119 39.5) (end 119 31.5) (stroke (width 0.05) (type default)) (layer "Edge.Cuts"))
 (gr_line (start 120 70.5) (end 119 70.5) (stroke (width 0.05) (type default)) (layer "Edge.Cuts"))
 (gr_line (start 113 19) (end 113 83) (stroke (width 0.05) (type default)) (layer "Edge.Cuts"))
 (gr_line (start 165 70.5) (end 164 70.5) (stroke (width 0.05) (type default)) (layer "Edge.Cuts"))
 (gr_line (start 132 83) (end 132 80) (stroke (width 0.05) (type default)) (layer "Edge.Cuts"))
 (gr_rect (start 149.496 53.848) (end 158.496 62.848) (stroke (width 0.05) (type default)) (fill none) (layer "Edge.Cuts"))
 (gr_line (start 165 31.5) (end 165 39.5) (stroke (width 0.05) (type default)) (layer "Edge.Cuts"))
 (gr_line (start 153.5 74) (end 153.5 73) (stroke (width 0.05) (type default)) (layer "Edge.Cuts"))
 (gr_line (start 130.5 73) (end 130.5 74) (stroke (width 0.05) (type default)) (layer "Edge.Cuts"))
 (gr_line (start 122.5 29) (end 122.5 28) (stroke (width 0.05) (type default)) (layer "Edge.Cuts"))
 (gr_line (start 153.5 28) (end 161.5 28) (stroke (width 0.05) (type default)) (layer "Edge.Cuts"))
 (gr_line (start 165 70.5) (end 164 70.5) (stroke (width 0.05) (type default)) (layer "Edge.Cuts"))
 (gr_circle (center 141.696 49.753) (end 147.946 49.753) (stroke (width 0.2) (type default)) (fill none) (layer "Edge.Cuts"))
 (gr_line (start 164 31.5) (end 165 31.5) (stroke (width 0.05) (type default)) (layer "Edge.Cuts"))
 (gr_line (start 119 62.5) (end 120 62.5) (stroke (width 0.05) (type default)) (layer "Edge.Cuts"))
 (gr_line (start 119 39.5) (end 119 31.5) (stroke (width 0.05) (type default)) (layer "Edge.Cuts"))
 (gr_circle (center 125 68) (end 125 66) (stroke (width 0.05) (type default)) (fill none) (layer "Edge.Cuts"))
 (gr_line (start 119 31.5) (end 120 31.5) (stroke (width 0.05) (type default)) (layer "Edge.Cuts"))
 (gr_line (start 161.5 74) (end 153.5 74) (stroke (width 0.05) (type default)) (layer "Edge.Cuts"))
 (gr_line (start 164 70.5) (end 164 62.5) (stroke (width 0.05) (type default)) (layer "Edge.Cuts"))
 (gr_line (start 120 31.5) (end 120 39.5) (stroke (width 0.05) (type default)) (layer "Edge.Cuts"))
 (gr_line (start 165 62.5) (end 165 70.5) (stroke (width 0.05) (type default)) (layer "Edge.Cuts"))
 (gr_line (start 120 31.5) (end 120 39.5) (stroke (width 0.05) (type default)) (layer "Edge.Cuts"))
 (gr_line (start 161.5 28) (end 161.5 29) (stroke (width 0.05) (type default)) (layer "Edge.Cuts"))
 (gr_line (start 122.5 74) (end 122.5 73) (stroke (width 0.05) (type default)) (layer "Edge.Cuts"))
 (gr_line (start 130.5 29) (end 122.5 29) (stroke (width 0.05) (type default)) (layer "Edge.Cuts"))
 (gr_line (start 171 83) (end 171 19) (stroke (width 0.05) (type default)) (layer "Edge.Cuts"))
 (gr_line (start 161.5 73) (end 161.5 74) (stroke (width 0.05) (type default)) (layer "Edge.Cuts"))
 (gr_line (start 132 83) (end 113 83) (stroke (width 0.05) (type default)) (layer "Edge.Cuts"))
 (gr_line (start 152 80) (end 152 83) (stroke (width 0.05) (type default)) (layer "Edge.Cuts"))
 (gr_line (start 119 70.5) (end 119 62.5) (stroke (width 0.05) (type default)) (layer "Edge.Cuts"))
 (gr_circle (center 159 34) (end 159 36) (stroke (width 0.05) (type default)) (fill none) (layer "Edge.Cuts"))
 (gr_line (start 119 62.5) (end 120 62.5) (stroke (width 0.05) (type default)) (layer "Edge.Cuts"))
 (gr_line (start 120 62.5) (end 120 70.5) (stroke (width 0.05) (type default)) (layer "Edge.Cuts"))
 (gr_line (start 132 80) (end 152 80) (stroke (width 0.05) (type default)) (layer "Edge.Cuts"))
 (gr_line (start 152 22) (end 132 22) (stroke (width 0.05) (type default)) (layer "Edge.Cuts"))
 (gr_line (start 165 39.5) (end 164 39.5) (stroke (width 0.05) (type default)) (layer "Edge.Cuts"))
 (gr_line (start 130.5 74) (end 122.5 74) (stroke (width 0.05) (type default)) (layer "Edge.Cuts"))
 (gr_line (start 161.5 29) (end 153.5 29) (stroke (width 0.05) (type default)) (layer "Edge.Cuts"))
 (gr_line (start 152 19) (end 152 22) (stroke (width 0.05) (type default)) (layer "Edge.Cuts"))
 (gr_line (start 164 70.5) (end 164 62.5) (stroke (width 0.05) (type default)) (layer "Edge.Cuts"))
 (gr_circle (center 159 34) (end 159 36) (stroke (width 0.05) (type default)) (fill none) (layer "Edge.Cuts"))
 (gr_line (start 153.5 28) (end 161.5 28) (stroke (width 0.05) (type default)) (layer "Edge.Cuts"))
 (gr_line (start 164 31.5) (end 165 31.5) (stroke (width 0.05) (type default)) (layer "Edge.Cuts"))
 (gr_line (start 153.5 73) (end 161.5 73) (stroke (width 0.05) (type default)) (layer "Edge.Cuts"))
 (gr_circle (center 159 68) (end 157 68) (stroke (width 0.05) (type default)) (fill none) (layer "Edge.Cuts"))
 (gr_line (start 122.5 74) (end 122.5 73) (stroke (width 0.05) (type default)) (layer "Edge.Cuts"))
 (gr_circle (center 159 68) (end 157 68) (stroke (width 0.05) (type default)) (fill none) (layer "Edge.Cuts"))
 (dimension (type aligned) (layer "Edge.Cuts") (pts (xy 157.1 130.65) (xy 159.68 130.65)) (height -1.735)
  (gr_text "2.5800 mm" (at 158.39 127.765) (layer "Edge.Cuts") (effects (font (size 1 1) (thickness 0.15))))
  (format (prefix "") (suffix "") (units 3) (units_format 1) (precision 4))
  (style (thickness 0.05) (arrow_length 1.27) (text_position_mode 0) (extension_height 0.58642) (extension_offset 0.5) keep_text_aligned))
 (segment (start 142.45 32.18) (end 135.4 32.18) (width 0.7) (layer "F.Cu") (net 8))
 (segment (start 135.4 32.18) (end 131.418 36.162) (width 0.7) (layer "F.Cu") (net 8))
 (segment (start 131.418 55.144) (end 131.568 55.294) (width 0.7) (layer "F.Cu") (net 8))
 (segment (start 131.568 55.294) (end 128.937 57.925) (width 0.7) (layer "F.Cu") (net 8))
 (segment (start 131.537 72.529) (end 138.791 72.529) (width 0.7) (layer "F.Cu") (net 8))
 (segment (start 131.418 36.162) (end 131.418 55.144) (width 0.7) (layer "F.Cu") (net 8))
 (segment (start 128.937 57.925) (end 128.937 69.929) (width 0.7) (layer "F.Cu") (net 8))
 (segment (start 128.937 69.929) (end 131.537 72.529) (width 0.7) (layer "F.Cu") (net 8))
 (segment (start 138.791 72.529) (end 142.1 69.22) (width 0.7) (layer "F.Cu") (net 8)))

